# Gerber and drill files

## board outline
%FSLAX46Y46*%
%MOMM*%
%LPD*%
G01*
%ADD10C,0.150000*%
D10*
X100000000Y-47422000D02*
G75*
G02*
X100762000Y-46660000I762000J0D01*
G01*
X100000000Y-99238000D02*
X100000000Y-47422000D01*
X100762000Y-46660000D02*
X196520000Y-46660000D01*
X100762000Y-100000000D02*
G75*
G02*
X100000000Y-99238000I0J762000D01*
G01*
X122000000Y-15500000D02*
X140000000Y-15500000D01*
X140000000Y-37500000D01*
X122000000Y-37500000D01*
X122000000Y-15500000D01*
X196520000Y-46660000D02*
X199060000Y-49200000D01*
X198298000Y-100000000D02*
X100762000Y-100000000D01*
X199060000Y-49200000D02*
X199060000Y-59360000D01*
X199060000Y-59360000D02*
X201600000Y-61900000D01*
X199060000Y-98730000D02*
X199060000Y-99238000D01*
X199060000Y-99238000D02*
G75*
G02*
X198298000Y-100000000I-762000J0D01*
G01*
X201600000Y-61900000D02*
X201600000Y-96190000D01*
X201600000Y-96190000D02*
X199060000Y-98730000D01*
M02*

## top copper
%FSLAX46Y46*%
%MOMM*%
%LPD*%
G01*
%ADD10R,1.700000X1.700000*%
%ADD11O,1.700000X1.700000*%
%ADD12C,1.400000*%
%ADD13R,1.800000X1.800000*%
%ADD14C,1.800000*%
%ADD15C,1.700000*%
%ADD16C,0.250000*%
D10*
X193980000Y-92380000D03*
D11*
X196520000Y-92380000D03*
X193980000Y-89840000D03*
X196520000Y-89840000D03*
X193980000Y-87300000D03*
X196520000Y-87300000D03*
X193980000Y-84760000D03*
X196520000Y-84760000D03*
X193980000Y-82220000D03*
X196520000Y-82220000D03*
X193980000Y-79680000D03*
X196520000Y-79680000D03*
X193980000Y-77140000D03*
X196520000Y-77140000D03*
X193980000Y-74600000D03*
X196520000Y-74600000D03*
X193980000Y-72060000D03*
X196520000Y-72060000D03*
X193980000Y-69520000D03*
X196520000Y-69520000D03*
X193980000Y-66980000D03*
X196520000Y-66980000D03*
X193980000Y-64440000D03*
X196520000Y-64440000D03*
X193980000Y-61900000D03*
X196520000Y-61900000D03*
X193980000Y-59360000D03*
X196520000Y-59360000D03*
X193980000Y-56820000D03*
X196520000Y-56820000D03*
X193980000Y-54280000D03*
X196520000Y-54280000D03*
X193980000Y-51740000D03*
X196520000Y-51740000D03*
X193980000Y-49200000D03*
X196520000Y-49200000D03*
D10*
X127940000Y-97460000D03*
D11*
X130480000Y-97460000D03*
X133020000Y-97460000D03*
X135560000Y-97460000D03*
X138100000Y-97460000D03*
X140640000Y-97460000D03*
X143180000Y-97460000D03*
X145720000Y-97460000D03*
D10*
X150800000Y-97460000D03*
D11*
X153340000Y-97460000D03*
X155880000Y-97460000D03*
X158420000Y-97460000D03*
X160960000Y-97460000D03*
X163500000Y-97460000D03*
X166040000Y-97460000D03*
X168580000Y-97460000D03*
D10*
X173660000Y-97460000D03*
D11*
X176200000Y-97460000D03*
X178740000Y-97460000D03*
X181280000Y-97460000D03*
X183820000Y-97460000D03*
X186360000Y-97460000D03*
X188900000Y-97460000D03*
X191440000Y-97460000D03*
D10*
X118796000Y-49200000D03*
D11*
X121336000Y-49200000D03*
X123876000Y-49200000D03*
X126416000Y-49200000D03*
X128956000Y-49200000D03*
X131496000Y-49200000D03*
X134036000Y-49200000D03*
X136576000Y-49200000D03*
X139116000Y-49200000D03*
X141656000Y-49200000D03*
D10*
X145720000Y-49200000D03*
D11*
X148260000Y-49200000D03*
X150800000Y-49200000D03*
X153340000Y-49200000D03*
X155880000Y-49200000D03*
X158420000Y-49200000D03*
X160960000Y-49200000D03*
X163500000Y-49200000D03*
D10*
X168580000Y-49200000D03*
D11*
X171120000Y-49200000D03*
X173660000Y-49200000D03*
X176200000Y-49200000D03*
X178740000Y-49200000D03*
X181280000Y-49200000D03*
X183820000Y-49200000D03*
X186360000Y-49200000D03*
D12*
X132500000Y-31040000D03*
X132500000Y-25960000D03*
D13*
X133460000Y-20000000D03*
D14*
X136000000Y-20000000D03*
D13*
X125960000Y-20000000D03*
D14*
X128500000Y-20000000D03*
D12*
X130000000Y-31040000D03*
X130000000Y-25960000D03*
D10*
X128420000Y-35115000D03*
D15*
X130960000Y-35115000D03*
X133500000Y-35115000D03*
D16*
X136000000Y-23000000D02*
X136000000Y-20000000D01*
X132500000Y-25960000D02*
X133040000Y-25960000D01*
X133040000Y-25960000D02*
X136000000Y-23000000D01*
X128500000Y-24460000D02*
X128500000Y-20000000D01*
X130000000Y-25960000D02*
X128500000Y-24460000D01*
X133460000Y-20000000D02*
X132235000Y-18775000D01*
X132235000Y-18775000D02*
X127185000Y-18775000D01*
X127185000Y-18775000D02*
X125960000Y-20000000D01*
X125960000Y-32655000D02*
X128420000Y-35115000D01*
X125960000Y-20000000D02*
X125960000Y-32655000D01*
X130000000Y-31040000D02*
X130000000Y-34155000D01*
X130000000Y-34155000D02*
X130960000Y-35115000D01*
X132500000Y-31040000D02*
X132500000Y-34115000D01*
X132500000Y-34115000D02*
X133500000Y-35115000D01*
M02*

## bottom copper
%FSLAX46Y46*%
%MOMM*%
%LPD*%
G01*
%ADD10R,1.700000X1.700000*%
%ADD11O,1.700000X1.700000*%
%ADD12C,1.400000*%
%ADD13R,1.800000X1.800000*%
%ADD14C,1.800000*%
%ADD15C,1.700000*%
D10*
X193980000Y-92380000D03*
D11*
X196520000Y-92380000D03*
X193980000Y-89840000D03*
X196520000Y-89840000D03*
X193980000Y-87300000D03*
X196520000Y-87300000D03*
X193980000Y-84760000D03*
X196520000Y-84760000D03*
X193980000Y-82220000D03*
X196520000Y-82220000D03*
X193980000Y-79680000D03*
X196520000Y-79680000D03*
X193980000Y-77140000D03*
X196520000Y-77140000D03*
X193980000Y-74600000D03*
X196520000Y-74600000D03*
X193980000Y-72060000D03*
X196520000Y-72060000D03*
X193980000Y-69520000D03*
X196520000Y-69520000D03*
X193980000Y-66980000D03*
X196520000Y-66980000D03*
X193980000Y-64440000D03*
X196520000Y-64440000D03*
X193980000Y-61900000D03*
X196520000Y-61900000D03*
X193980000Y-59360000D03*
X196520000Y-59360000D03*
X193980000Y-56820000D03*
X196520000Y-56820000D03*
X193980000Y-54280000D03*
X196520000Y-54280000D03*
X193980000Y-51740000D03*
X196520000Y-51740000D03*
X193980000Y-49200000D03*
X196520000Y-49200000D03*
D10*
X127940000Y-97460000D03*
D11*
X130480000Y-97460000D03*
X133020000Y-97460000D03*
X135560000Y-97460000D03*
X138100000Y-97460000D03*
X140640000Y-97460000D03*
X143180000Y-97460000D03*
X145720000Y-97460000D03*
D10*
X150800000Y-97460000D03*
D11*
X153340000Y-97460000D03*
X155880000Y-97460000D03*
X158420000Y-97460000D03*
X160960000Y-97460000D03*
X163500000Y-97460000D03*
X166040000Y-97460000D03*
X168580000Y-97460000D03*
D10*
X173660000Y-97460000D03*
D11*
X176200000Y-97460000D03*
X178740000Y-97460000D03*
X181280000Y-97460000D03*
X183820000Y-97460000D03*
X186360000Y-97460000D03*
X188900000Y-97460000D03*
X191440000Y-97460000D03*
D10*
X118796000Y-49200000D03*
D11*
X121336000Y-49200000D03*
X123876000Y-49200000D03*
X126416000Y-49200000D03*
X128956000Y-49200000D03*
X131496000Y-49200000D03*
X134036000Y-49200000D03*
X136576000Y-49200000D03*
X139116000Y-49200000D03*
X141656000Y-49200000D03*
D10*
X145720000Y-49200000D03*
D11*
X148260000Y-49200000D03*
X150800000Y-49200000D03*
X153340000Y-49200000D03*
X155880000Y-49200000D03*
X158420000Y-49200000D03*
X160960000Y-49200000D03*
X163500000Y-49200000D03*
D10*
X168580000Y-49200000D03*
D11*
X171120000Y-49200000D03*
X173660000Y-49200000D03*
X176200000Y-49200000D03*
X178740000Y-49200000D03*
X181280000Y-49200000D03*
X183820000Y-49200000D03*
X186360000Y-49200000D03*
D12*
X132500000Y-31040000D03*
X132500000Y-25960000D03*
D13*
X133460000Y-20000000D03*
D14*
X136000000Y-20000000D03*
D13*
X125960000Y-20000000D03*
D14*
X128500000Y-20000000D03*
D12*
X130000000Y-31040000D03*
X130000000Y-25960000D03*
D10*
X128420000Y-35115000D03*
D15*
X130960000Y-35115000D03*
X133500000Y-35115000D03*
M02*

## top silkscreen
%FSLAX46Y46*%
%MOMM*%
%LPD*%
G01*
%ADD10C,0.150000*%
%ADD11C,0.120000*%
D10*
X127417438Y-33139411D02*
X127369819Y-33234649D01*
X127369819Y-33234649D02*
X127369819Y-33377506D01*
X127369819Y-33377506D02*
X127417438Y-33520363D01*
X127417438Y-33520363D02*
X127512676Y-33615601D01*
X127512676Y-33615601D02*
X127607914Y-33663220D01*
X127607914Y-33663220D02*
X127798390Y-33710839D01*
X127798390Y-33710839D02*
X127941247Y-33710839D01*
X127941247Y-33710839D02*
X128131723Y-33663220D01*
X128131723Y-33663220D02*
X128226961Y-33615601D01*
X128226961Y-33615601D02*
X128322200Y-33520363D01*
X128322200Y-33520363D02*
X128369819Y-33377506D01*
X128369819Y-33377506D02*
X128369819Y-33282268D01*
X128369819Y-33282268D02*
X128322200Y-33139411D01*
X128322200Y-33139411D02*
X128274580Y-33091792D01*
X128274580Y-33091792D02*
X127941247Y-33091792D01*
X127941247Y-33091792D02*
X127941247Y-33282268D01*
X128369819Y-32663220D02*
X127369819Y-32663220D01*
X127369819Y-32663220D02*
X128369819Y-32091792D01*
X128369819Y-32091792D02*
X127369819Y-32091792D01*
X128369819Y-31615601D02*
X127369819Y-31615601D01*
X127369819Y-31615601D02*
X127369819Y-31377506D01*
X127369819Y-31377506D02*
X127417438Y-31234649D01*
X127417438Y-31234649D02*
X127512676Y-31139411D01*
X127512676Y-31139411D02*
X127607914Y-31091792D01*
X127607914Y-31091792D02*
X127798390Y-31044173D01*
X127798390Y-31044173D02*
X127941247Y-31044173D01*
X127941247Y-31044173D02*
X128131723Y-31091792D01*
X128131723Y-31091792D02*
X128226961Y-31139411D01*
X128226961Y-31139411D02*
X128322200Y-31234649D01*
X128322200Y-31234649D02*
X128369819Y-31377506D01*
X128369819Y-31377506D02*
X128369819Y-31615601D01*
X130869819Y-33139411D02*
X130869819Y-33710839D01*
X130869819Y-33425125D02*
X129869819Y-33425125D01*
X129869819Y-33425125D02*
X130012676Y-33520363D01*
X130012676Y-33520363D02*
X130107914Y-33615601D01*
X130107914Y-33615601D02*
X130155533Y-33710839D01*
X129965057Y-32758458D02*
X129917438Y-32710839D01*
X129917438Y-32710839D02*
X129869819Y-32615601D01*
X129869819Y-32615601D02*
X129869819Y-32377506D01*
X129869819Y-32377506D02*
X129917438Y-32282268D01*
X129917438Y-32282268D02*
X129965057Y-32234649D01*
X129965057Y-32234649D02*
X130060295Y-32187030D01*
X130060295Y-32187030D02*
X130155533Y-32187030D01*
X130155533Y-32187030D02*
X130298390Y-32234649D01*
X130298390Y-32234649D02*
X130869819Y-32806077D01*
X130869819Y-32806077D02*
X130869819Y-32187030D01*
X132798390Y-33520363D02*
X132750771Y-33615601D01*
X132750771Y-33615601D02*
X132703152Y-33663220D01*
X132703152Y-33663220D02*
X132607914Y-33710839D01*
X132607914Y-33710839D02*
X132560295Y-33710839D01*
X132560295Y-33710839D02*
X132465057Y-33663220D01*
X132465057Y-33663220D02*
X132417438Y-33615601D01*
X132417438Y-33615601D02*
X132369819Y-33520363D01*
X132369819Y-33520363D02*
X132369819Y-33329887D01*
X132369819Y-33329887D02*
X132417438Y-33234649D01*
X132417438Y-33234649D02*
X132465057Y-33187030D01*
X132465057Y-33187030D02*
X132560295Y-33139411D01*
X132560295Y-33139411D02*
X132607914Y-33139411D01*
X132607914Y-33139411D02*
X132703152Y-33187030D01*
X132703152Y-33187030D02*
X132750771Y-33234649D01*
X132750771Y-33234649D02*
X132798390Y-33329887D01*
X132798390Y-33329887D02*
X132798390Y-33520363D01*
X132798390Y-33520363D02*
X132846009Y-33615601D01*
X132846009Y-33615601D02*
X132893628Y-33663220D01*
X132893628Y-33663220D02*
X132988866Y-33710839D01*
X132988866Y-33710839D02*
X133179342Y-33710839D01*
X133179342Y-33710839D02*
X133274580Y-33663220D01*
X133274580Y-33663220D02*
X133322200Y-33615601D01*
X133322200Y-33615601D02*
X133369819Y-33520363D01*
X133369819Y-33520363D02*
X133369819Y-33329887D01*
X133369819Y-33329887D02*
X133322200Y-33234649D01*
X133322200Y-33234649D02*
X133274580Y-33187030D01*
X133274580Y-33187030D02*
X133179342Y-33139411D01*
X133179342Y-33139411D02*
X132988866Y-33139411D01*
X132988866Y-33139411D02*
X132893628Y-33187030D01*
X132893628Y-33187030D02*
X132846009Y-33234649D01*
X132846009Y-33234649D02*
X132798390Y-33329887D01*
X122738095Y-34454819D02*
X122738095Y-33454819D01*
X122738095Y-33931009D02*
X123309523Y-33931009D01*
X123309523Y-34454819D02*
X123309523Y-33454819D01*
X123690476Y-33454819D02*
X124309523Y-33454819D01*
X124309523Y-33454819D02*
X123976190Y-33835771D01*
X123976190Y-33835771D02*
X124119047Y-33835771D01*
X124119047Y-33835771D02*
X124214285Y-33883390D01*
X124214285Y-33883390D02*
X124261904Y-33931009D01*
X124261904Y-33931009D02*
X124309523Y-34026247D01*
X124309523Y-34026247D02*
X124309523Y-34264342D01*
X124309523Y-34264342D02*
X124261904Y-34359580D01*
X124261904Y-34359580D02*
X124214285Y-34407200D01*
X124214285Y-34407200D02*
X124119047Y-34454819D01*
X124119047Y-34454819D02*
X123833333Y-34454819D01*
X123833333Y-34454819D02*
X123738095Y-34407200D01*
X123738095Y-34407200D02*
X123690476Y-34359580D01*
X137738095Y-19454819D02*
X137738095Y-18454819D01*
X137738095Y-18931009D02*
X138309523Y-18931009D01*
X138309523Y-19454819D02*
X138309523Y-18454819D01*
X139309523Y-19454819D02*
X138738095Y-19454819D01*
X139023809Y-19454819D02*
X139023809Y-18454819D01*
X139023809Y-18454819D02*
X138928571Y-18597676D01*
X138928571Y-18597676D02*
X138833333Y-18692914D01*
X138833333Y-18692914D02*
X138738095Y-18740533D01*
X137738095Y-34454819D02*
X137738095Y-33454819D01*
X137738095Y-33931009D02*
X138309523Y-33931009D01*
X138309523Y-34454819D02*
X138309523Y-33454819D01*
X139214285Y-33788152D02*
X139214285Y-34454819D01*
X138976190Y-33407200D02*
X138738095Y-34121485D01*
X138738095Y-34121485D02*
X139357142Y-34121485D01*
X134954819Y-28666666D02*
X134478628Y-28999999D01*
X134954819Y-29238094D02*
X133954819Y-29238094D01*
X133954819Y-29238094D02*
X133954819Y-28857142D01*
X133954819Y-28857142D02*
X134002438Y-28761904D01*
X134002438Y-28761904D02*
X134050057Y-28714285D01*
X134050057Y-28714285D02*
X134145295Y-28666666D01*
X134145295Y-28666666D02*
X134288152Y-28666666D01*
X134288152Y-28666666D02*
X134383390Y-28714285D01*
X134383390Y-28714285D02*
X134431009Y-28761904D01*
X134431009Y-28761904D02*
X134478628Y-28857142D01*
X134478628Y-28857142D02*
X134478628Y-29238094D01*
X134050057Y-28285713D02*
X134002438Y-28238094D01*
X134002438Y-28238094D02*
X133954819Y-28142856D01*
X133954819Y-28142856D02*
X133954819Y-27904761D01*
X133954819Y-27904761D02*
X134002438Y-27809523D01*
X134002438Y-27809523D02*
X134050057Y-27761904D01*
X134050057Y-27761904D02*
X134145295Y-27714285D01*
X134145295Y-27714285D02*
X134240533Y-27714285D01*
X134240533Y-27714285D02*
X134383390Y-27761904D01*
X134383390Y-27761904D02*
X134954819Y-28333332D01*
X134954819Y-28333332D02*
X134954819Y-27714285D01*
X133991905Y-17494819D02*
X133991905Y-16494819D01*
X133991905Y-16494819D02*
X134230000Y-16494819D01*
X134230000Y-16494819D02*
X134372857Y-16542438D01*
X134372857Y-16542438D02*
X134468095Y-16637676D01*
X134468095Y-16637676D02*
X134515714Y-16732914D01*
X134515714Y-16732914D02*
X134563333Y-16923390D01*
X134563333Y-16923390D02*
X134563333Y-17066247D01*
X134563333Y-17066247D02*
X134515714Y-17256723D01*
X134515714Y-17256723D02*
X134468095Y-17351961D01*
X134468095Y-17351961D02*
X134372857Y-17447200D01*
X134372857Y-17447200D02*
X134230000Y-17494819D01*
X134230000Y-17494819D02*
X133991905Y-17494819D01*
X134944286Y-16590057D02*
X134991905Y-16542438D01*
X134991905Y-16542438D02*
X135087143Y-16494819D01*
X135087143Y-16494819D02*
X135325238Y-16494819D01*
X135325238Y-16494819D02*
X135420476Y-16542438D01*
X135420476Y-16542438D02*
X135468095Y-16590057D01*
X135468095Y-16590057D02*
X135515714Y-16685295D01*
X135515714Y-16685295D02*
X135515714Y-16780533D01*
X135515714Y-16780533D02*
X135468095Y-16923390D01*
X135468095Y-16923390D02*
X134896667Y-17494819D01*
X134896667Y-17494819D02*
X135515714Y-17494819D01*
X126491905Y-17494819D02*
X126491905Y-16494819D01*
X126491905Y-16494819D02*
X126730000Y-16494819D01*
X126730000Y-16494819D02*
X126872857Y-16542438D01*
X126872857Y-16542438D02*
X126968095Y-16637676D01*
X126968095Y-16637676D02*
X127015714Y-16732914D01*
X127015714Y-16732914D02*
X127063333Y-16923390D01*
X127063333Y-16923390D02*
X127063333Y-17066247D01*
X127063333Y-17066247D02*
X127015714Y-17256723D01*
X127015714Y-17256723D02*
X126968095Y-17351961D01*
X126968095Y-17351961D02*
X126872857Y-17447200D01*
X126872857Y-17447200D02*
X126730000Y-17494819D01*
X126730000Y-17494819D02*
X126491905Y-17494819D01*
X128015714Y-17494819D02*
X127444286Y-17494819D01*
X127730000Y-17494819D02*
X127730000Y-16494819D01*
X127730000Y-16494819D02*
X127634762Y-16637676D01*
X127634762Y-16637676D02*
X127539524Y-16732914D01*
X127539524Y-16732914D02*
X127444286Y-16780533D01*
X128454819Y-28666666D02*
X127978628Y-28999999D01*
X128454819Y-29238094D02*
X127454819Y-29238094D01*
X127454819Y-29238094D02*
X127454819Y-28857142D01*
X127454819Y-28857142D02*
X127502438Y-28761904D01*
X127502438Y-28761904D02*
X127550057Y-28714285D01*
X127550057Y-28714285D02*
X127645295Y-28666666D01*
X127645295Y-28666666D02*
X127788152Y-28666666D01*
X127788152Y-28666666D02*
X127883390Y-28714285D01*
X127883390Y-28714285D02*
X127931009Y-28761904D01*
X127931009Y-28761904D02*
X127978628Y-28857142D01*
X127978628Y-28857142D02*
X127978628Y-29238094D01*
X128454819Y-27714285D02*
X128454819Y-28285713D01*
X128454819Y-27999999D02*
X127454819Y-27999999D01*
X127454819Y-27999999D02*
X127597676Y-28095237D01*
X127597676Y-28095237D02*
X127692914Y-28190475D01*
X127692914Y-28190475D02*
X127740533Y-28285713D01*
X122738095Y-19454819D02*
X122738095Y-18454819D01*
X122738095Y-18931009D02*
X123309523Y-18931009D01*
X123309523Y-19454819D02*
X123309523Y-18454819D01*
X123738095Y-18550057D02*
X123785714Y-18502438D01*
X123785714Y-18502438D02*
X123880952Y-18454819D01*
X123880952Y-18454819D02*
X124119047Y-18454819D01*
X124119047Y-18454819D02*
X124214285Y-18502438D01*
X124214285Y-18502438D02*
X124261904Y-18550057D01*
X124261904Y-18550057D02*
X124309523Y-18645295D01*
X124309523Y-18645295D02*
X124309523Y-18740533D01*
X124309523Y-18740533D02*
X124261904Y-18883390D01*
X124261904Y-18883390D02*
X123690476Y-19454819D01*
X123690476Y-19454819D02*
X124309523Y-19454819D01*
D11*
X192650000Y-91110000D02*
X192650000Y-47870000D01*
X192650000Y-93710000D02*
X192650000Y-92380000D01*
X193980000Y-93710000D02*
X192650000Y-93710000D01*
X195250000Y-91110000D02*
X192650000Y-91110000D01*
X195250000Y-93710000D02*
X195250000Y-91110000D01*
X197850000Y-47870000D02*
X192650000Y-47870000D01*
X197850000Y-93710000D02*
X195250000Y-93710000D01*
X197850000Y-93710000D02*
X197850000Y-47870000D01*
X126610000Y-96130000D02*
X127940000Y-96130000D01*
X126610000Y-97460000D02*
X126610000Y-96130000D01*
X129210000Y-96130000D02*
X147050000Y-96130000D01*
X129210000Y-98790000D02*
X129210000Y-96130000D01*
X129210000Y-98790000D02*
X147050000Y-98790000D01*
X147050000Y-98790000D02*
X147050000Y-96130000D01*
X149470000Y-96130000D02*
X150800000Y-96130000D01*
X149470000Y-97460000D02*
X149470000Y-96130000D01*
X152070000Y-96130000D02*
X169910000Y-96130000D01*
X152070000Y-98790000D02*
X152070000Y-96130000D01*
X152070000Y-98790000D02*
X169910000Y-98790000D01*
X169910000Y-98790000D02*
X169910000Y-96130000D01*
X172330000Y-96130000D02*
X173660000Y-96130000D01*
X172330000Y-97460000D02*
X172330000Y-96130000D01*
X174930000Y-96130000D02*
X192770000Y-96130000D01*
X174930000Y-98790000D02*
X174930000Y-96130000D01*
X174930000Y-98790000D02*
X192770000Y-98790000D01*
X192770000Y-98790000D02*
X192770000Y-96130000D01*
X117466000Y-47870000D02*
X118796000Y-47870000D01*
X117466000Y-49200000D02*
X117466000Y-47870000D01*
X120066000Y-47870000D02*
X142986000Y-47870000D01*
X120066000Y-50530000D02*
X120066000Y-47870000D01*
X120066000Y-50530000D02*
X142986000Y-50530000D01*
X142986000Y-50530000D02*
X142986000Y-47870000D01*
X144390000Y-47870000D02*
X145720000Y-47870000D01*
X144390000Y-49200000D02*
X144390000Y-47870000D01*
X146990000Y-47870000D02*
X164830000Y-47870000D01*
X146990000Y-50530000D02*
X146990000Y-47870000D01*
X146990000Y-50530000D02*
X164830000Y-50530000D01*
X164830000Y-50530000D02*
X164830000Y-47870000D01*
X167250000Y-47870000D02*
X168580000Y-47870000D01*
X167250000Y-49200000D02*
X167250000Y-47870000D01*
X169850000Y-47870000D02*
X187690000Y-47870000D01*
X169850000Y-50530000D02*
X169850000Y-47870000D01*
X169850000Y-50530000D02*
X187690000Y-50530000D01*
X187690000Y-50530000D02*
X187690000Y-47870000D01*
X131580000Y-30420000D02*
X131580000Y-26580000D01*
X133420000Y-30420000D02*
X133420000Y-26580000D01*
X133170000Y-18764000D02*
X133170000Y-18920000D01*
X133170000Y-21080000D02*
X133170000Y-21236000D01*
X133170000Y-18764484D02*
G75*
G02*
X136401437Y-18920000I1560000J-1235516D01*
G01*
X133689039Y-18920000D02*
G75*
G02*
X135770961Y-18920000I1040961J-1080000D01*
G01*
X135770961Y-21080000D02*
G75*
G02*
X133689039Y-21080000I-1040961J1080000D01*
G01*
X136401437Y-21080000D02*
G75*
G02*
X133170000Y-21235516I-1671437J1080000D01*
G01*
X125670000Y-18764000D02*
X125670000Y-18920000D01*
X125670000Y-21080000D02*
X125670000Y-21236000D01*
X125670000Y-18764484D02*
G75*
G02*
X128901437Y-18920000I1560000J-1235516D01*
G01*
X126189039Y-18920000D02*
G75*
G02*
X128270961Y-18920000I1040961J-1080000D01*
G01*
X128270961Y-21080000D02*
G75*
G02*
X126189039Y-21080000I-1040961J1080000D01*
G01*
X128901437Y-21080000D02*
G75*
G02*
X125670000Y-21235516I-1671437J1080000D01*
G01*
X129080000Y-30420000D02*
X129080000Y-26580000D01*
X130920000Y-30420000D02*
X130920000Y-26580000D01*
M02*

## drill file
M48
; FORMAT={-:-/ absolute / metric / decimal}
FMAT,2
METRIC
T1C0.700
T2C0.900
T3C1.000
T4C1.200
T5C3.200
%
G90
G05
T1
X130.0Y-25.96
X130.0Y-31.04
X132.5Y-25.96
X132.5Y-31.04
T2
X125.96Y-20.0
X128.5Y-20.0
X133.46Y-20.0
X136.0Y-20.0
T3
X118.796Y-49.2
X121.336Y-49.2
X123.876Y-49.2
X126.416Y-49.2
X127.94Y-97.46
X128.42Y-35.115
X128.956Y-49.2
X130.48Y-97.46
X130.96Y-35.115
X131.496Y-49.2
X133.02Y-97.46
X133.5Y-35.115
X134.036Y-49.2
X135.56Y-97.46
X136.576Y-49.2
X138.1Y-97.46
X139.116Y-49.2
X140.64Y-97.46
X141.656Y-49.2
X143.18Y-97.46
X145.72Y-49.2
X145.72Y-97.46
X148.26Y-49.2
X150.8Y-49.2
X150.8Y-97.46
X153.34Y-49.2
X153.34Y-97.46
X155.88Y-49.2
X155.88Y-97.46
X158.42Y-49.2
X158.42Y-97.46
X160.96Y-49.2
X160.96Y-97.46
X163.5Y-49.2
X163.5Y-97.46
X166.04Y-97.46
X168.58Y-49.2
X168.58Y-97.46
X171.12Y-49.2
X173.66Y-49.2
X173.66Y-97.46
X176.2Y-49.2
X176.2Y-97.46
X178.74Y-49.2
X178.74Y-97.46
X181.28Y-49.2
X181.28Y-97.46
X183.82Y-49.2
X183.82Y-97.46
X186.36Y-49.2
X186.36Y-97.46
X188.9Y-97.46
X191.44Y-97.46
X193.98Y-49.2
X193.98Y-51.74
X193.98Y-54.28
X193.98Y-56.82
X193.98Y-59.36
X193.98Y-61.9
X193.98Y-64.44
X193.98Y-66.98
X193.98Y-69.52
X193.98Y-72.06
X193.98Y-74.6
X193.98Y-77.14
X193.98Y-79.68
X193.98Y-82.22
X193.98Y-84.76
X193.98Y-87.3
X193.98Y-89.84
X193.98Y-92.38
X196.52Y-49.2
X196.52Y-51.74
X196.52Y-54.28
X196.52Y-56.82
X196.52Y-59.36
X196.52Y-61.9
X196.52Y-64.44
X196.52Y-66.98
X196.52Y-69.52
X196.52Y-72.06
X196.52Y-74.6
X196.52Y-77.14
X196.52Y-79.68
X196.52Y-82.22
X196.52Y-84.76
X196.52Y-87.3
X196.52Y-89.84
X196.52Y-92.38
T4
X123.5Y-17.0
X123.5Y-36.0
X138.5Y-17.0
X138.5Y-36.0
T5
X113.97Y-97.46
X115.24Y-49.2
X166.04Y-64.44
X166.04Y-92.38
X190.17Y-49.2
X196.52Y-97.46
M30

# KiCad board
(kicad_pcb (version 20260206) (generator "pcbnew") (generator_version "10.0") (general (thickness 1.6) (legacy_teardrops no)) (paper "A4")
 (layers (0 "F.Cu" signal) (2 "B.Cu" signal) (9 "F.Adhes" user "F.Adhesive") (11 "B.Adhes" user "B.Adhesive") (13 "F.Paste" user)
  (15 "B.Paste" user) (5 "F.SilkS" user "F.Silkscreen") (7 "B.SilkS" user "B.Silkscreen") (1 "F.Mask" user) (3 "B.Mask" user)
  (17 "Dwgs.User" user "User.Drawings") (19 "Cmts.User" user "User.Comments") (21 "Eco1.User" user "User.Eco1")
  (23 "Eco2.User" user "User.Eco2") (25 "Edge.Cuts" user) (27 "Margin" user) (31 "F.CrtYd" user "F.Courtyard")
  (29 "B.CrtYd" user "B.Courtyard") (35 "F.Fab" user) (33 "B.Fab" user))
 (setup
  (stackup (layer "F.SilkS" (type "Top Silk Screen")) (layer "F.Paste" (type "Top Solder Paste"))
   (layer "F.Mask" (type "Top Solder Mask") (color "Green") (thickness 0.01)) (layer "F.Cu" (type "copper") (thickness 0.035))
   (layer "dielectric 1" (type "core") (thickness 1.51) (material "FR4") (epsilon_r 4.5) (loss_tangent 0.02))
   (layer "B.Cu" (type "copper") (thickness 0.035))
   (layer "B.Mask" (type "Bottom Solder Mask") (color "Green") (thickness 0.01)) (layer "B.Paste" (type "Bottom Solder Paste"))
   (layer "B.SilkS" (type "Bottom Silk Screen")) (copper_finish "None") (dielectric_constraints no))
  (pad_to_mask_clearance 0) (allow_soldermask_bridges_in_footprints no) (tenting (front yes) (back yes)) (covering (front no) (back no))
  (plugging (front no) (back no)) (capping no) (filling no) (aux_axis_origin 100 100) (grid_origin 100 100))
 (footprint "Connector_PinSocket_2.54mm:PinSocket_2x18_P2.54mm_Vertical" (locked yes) (layer "F.Cu") (at 193.98 92.38 180)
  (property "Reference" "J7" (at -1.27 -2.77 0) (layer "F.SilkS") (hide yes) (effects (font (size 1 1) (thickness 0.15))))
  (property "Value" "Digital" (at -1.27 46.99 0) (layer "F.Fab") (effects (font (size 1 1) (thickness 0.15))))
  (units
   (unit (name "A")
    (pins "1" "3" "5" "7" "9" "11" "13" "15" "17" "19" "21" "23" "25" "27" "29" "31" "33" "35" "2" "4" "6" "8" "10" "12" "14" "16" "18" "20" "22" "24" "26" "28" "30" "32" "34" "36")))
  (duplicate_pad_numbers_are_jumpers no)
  (fp_line (start 1.33 1.27) (end 1.33 44.51) (stroke (width 0.12) (type solid)) (layer "F.SilkS"))
  (fp_line (start 1.33 -1.33) (end 1.33 0) (stroke (width 0.12) (type solid)) (layer "F.SilkS"))
  (fp_line (start 0 -1.33) (end 1.33 -1.33) (stroke (width 0.12) (type solid)) (layer "F.SilkS"))
  (fp_line (start -1.27 1.27) (end 1.33 1.27) (stroke (width 0.12) (type solid)) (layer "F.SilkS"))
  (fp_line (start -1.27 -1.33) (end -1.27 1.27) (stroke (width 0.12) (type solid)) (layer "F.SilkS"))
  (fp_line (start -3.87 44.51) (end 1.33 44.51) (stroke (width 0.12) (type solid)) (layer "F.SilkS"))
  (fp_line (start -3.87 -1.33) (end -1.27 -1.33) (stroke (width 0.12) (type solid)) (layer "F.SilkS"))
  (fp_line (start -3.87 -1.33) (end -3.87 44.51) (stroke (width 0.12) (type solid)) (layer "F.SilkS"))
  (pad "1" thru_hole rect (at 0 0 180) (size 1.7 1.7) (drill 1) (layers "*.Cu" "*.Mask") (remove_unused_layers no) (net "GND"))
  (pad "2" thru_hole oval (at -2.54 0 180) (size 1.7 1.7) (drill 1) (layers "*.Cu" "*.Mask") (remove_unused_layers no) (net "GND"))
  (pad "3" thru_hole oval (at 0 2.54 180) (size 1.7 1.7) (drill 1) (layers "*.Cu" "*.Mask") (remove_unused_layers no) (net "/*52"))
  (pad "4" thru_hole oval (at -2.54 2.54 180) (size 1.7 1.7) (drill 1) (layers "*.Cu" "*.Mask") (remove_unused_layers no) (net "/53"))
  (pad "5" thru_hole oval (at 0 5.08 180) (size 1.7 1.7) (drill 1) (layers "*.Cu" "*.Mask") (remove_unused_layers no) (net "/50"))
  (pad "6" thru_hole oval (at -2.54 5.08 180) (size 1.7 1.7) (drill 1) (layers "*.Cu" "*.Mask") (remove_unused_layers no) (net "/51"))
  (pad "7" thru_hole oval (at 0 7.62 180) (size 1.7 1.7) (drill 1) (layers "*.Cu" "*.Mask") (remove_unused_layers no) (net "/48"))
  (pad "8" thru_hole oval (at -2.54 7.62 180) (size 1.7 1.7) (drill 1) (layers "*.Cu" "*.Mask") (remove_unused_layers no) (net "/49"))
  (pad "9" thru_hole oval (at 0 10.16 180) (size 1.7 1.7) (drill 1) (layers "*.Cu" "*.Mask") (remove_unused_layers no) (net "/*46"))
  (pad "10" thru_hole oval (at -2.54 10.16 180) (size 1.7 1.7) (drill 1) (layers "*.Cu" "*.Mask") (remove_unused_layers no) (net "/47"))
  (pad "11" thru_hole oval (at 0 12.7 180) (size 1.7 1.7) (drill 1) (layers "*.Cu" "*.Mask") (remove_unused_layers no) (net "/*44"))
  (pad "12" thru_hole oval (at -2.54 12.7 180) (size 1.7 1.7) (drill 1) (layers "*.Cu" "*.Mask") (remove_unused_layers no) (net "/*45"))
  (pad "13" thru_hole oval (at 0 15.24 180) (size 1.7 1.7) (drill 1) (layers "*.Cu" "*.Mask") (remove_unused_layers no) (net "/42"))
  (pad "14" thru_hole oval (at -2.54 15.24 180) (size 1.7 1.7) (drill 1) (layers "*.Cu" "*.Mask") (remove_unused_layers no) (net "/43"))
  (pad "15" thru_hole oval (at 0 17.78 180) (size 1.7 1.7) (drill 1) (layers "*.Cu" "*.Mask") (remove_unused_layers no) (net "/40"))
  (pad "16" thru_hole oval (at -2.54 17.78 180) (size 1.7 1.7) (drill 1) (layers "*.Cu" "*.Mask") (remove_unused_layers no) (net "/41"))
  (pad "17" thru_hole oval (at 0 20.32 180) (size 1.7 1.7) (drill 1) (layers "*.Cu" "*.Mask") (remove_unused_layers no) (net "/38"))
  (pad "18" thru_hole oval (at -2.54 20.32 180) (size 1.7 1.7) (drill 1) (layers "*.Cu" "*.Mask") (remove_unused_layers no) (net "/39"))
  (pad "19" thru_hole oval (at 0 22.86 180) (size 1.7 1.7) (drill 1) (layers "*.Cu" "*.Mask") (remove_unused_layers no) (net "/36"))
  (pad "20" thru_hole oval (at -2.54 22.86 180) (size 1.7 1.7) (drill 1) (layers "*.Cu" "*.Mask") (remove_unused_layers no) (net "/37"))
  (pad "21" thru_hole oval (at 0 25.4 180) (size 1.7 1.7) (drill 1) (layers "*.Cu" "*.Mask") (remove_unused_layers no) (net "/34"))
  (pad "22" thru_hole oval (at -2.54 25.4 180) (size 1.7 1.7) (drill 1) (layers "*.Cu" "*.Mask") (remove_unused_layers no) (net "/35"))
  (pad "23" thru_hole oval (at 0 27.94 180) (size 1.7 1.7) (drill 1) (layers "*.Cu" "*.Mask") (remove_unused_layers no) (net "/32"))
  (pad "24" thru_hole oval (at -2.54 27.94 180) (size 1.7 1.7) (drill 1) (layers "*.Cu" "*.Mask") (remove_unused_layers no) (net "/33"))
  (pad "25" thru_hole oval (at 0 30.48 180) (size 1.7 1.7) (drill 1) (layers "*.Cu" "*.Mask") (remove_unused_layers no) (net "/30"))
  (pad "26" thru_hole oval (at -2.54 30.48 180) (size 1.7 1.7) (drill 1) (layers "*.Cu" "*.Mask") (remove_unused_layers no) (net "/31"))
  (pad "27" thru_hole oval (at 0 33.02 180) (size 1.7 1.7) (drill 1) (layers "*.Cu" "*.Mask") (remove_unused_layers no) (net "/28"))
  (pad "28" thru_hole oval (at -2.54 33.02 180) (size 1.7 1.7) (drill 1) (layers "*.Cu" "*.Mask") (remove_unused_layers no) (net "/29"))
  (pad "29" thru_hole oval (at 0 35.56 180) (size 1.7 1.7) (drill 1) (layers "*.Cu" "*.Mask") (remove_unused_layers no) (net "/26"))
  (pad "30" thru_hole oval (at -2.54 35.56 180) (size 1.7 1.7) (drill 1) (layers "*.Cu" "*.Mask") (remove_unused_layers no) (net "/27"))
  (pad "31" thru_hole oval (at 0 38.1 180) (size 1.7 1.7) (drill 1) (layers "*.Cu" "*.Mask") (remove_unused_layers no) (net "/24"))
  (pad "32" thru_hole oval (at -2.54 38.1 180) (size 1.7 1.7) (drill 1) (layers "*.Cu" "*.Mask") (remove_unused_layers no) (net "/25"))
  (pad "33" thru_hole oval (at 0 40.64 180) (size 1.7 1.7) (drill 1) (layers "*.Cu" "*.Mask") (remove_unused_layers no) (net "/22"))
  (pad "34" thru_hole oval (at -2.54 40.64 180) (size 1.7 1.7) (drill 1) (layers "*.Cu" "*.Mask") (remove_unused_layers no) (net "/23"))
  (pad "35" thru_hole oval (at 0 43.18 180) (size 1.7 1.7) (drill 1) (layers "*.Cu" "*.Mask") (remove_unused_layers no) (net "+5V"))
  (pad "36" thru_hole oval (at -2.54 43.18 180) (size 1.7 1.7) (drill 1) (layers "*.Cu" "*.Mask") (remove_unused_layers no) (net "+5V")))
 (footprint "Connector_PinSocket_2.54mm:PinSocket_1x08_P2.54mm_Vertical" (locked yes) (layer "F.Cu") (at 127.94 97.46 90)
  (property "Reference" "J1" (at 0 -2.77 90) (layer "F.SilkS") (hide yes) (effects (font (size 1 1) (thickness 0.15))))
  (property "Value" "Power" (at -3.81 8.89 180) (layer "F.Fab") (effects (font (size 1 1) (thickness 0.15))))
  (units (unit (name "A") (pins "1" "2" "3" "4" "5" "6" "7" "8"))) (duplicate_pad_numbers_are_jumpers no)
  (fp_line (start 1.33 -1.33) (end 1.33 0) (stroke (width 0.12) (type solid)) (layer "F.SilkS"))
  (fp_line (start 0 -1.33) (end 1.33 -1.33) (stroke (width 0.12) (type solid)) (layer "F.SilkS"))
  (fp_line (start 1.33 1.27) (end 1.33 19.11) (stroke (width 0.12) (type solid)) (layer "F.SilkS"))
  (fp_line (start -1.33 1.27) (end 1.33 1.27) (stroke (width 0.12) (type solid)) (layer "F.SilkS"))
  (fp_line (start -1.33 1.27) (end -1.33 19.11) (stroke (width 0.12) (type solid)) (layer "F.SilkS"))
  (fp_line (start -1.33 19.11) (end 1.33 19.11) (stroke (width 0.12) (type solid)) (layer "F.SilkS"))
  (pad "1" thru_hole rect (at 0 0 90) (size 1.7 1.7) (drill 1) (layers "*.Cu" "*.Mask") (remove_unused_layers no)
   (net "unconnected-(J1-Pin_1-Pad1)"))
  (pad "2" thru_hole oval (at 0 2.54 90) (size 1.7 1.7) (drill 1) (layers "*.Cu" "*.Mask") (remove_unused_layers no) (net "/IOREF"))
  (pad "3" thru_hole oval (at 0 5.08 90) (size 1.7 1.7) (drill 1) (layers "*.Cu" "*.Mask") (remove_unused_layers no) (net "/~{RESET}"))
  (pad "4" thru_hole oval (at 0 7.62 90) (size 1.7 1.7) (drill 1) (layers "*.Cu" "*.Mask") (remove_unused_layers no) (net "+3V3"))
  (pad "5" thru_hole oval (at 0 10.16 90) (size 1.7 1.7) (drill 1) (layers "*.Cu" "*.Mask") (remove_unused_layers no) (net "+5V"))
  (pad "6" thru_hole oval (at 0 12.7 90) (size 1.7 1.7) (drill 1) (layers "*.Cu" "*.Mask") (remove_unused_layers no) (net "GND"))
  (pad "7" thru_hole oval (at 0 15.24 90) (size 1.7 1.7) (drill 1) (layers "*.Cu" "*.Mask") (remove_unused_layers no) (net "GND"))
  (pad "8" thru_hole oval (at 0 17.78 90) (size 1.7 1.7) (drill 1) (layers "*.Cu" "*.Mask") (remove_unused_layers no) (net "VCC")))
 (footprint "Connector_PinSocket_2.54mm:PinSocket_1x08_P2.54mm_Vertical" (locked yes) (layer "F.Cu") (at 150.8 97.46 90)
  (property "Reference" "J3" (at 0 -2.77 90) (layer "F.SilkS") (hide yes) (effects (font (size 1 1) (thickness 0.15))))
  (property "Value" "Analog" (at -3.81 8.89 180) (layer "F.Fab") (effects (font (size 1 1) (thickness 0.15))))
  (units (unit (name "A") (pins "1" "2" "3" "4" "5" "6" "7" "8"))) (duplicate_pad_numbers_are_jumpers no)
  (fp_line (start 1.33 -1.33) (end 1.33 0) (stroke (width 0.12) (type solid)) (layer "F.SilkS"))
  (fp_line (start 0 -1.33) (end 1.33 -1.33) (stroke (width 0.12) (type solid)) (layer "F.SilkS"))
  (fp_line (start 1.33 1.27) (end 1.33 19.11) (stroke (width 0.12) (type solid)) (layer "F.SilkS"))
  (fp_line (start -1.33 1.27) (end 1.33 1.27) (stroke (width 0.12) (type solid)) (layer "F.SilkS"))
  (fp_line (start -1.33 1.27) (end -1.33 19.11) (stroke (width 0.12) (type solid)) (layer "F.SilkS"))
  (fp_line (start -1.33 19.11) (end 1.33 19.11) (stroke (width 0.12) (type solid)) (layer "F.SilkS"))
  (pad "1" thru_hole rect (at 0 0 90) (size 1.7 1.7) (drill 1) (layers "*.Cu" "*.Mask") (remove_unused_layers no) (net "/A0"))
  (pad "2" thru_hole oval (at 0 2.54 90) (size 1.7 1.7) (drill 1) (layers "*.Cu" "*.Mask") (remove_unused_layers no) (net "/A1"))
  (pad "3" thru_hole oval (at 0 5.08 90) (size 1.7 1.7) (drill 1) (layers "*.Cu" "*.Mask") (remove_unused_layers no) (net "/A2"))
  (pad "4" thru_hole oval (at 0 7.62 90) (size 1.7 1.7) (drill 1) (layers "*.Cu" "*.Mask") (remove_unused_layers no) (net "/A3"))
  (pad "5" thru_hole oval (at 0 10.16 90) (size 1.7 1.7) (drill 1) (layers "*.Cu" "*.Mask") (remove_unused_layers no) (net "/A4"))
  (pad "6" thru_hole oval (at 0 12.7 90) (size 1.7 1.7) (drill 1) (layers "*.Cu" "*.Mask") (remove_unused_layers no) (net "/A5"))
  (pad "7" thru_hole oval (at 0 15.24 90) (size 1.7 1.7) (drill 1) (layers "*.Cu" "*.Mask") (remove_unused_layers no) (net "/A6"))
  (pad "8" thru_hole oval (at 0 17.78 90) (size 1.7 1.7) (drill 1) (layers "*.Cu" "*.Mask") (remove_unused_layers no) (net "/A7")))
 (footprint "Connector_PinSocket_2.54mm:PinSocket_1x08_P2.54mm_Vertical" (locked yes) (layer "F.Cu") (at 173.66 97.46 90)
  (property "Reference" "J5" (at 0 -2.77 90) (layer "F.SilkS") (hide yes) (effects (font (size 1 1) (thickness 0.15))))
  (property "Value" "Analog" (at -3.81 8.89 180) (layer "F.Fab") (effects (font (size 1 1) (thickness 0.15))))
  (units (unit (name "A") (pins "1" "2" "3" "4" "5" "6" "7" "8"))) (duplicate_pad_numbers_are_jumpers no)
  (fp_line (start 1.33 -1.33) (end 1.33 0) (stroke (width 0.12) (type solid)) (layer "F.SilkS"))
  (fp_line (start 0 -1.33) (end 1.33 -1.33) (stroke (width 0.12) (type solid)) (layer "F.SilkS"))
  (fp_line (start 1.33 1.27) (end 1.33 19.11) (stroke (width 0.12) (type solid)) (layer "F.SilkS"))
  (fp_line (start -1.33 1.27) (end 1.33 1.27) (stroke (width 0.12) (type solid)) (layer "F.SilkS"))
  (fp_line (start -1.33 1.27) (end -1.33 19.11) (stroke (width 0.12) (type solid)) (layer "F.SilkS"))
  (fp_line (start -1.33 19.11) (end 1.33 19.11) (stroke (width 0.12) (type solid)) (layer "F.SilkS"))
  (pad "1" thru_hole rect (at 0 0 90) (size 1.7 1.7) (drill 1) (layers "*.Cu" "*.Mask") (remove_unused_layers no) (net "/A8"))
  (pad "2" thru_hole oval (at 0 2.54 90) (size 1.7 1.7) (drill 1) (layers "*.Cu" "*.Mask") (remove_unused_layers no) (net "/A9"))
  (pad "3" thru_hole oval (at 0 5.08 90) (size 1.7 1.7) (drill 1) (layers "*.Cu" "*.Mask") (remove_unused_layers no) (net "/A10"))
  (pad "4" thru_hole oval (at 0 7.62 90) (size 1.7 1.7) (drill 1) (layers "*.Cu" "*.Mask") (remove_unused_layers no) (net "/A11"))
  (pad "5" thru_hole oval (at 0 10.16 90) (size 1.7 1.7) (drill 1) (layers "*.Cu" "*.Mask") (remove_unused_layers no) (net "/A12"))
  (pad "6" thru_hole oval (at 0 12.7 90) (size 1.7 1.7) (drill 1) (layers "*.Cu" "*.Mask") (remove_unused_layers no) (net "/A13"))
  (pad "7" thru_hole oval (at 0 15.24 90) (size 1.7 1.7) (drill 1) (layers "*.Cu" "*.Mask") (remove_unused_layers no) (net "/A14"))
  (pad "8" thru_hole oval (at 0 17.78 90) (size 1.7 1.7) (drill 1) (layers "*.Cu" "*.Mask") (remove_unused_layers no) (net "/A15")))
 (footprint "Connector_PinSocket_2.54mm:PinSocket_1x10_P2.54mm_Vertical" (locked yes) (layer "F.Cu") (at 118.796 49.2 90)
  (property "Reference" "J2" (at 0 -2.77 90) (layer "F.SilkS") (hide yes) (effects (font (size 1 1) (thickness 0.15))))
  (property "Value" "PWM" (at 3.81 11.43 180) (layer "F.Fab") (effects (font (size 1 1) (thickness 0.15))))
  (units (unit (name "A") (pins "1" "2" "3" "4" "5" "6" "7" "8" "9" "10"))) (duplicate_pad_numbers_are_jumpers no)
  (fp_line (start 1.33 -1.33) (end 1.33 0) (stroke (width 0.12) (type solid)) (layer "F.SilkS"))
  (fp_line (start 0 -1.33) (end 1.33 -1.33) (stroke (width 0.12) (type solid)) (layer "F.SilkS"))
  (fp_line (start 1.33 1.27) (end 1.33 24.19) (stroke (width 0.12) (type solid)) (layer "F.SilkS"))
  (fp_line (start -1.33 1.27) (end 1.33 1.27) (stroke (width 0.12) (type solid)) (layer "F.SilkS"))
  (fp_line (start -1.33 1.27) (end -1.33 24.19) (stroke (width 0.12) (type solid)) (layer "F.SilkS"))
  (fp_line (start -1.33 24.19) (end 1.33 24.19) (stroke (width 0.12) (type solid)) (layer "F.SilkS"))
  (pad "1" thru_hole rect (at 0 0 90) (size 1.7 1.7) (drill 1) (layers "*.Cu" "*.Mask") (remove_unused_layers no) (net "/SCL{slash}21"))
  (pad "2" thru_hole oval (at 0 2.54 90) (size 1.7 1.7) (drill 1) (layers "*.Cu" "*.Mask") (remove_unused_layers no) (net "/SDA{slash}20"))
  (pad "3" thru_hole oval (at 0 5.08 90) (size 1.7 1.7) (drill 1) (layers "*.Cu" "*.Mask") (remove_unused_layers no) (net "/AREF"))
  (pad "4" thru_hole oval (at 0 7.62 90) (size 1.7 1.7) (drill 1) (layers "*.Cu" "*.Mask") (remove_unused_layers no) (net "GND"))
  (pad "5" thru_hole oval (at 0 10.16 90) (size 1.7 1.7) (drill 1) (layers "*.Cu" "*.Mask") (remove_unused_layers no) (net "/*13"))
  (pad "6" thru_hole oval (at 0 12.7 90) (size 1.7 1.7) (drill 1) (layers "*.Cu" "*.Mask") (remove_unused_layers no)
   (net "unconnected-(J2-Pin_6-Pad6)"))
  (pad "7" thru_hole oval (at 0 15.24 90) (size 1.7 1.7) (drill 1) (layers "*.Cu" "*.Mask") (remove_unused_layers no) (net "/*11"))
  (pad "8" thru_hole oval (at 0 17.78 90) (size 1.7 1.7) (drill 1) (layers "*.Cu" "*.Mask") (remove_unused_layers no)
   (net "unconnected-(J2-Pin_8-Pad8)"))
  (pad "9" thru_hole oval (at 0 20.32 90) (size 1.7 1.7) (drill 1) (layers "*.Cu" "*.Mask") (remove_unused_layers no) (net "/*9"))
  (pad "10" thru_hole oval (at 0 22.86 90) (size 1.7 1.7) (drill 1) (layers "*.Cu" "*.Mask") (remove_unused_layers no)
   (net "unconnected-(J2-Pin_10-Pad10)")))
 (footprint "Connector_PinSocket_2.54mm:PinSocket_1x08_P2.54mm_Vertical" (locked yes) (layer "F.Cu") (at 145.72 49.2 90)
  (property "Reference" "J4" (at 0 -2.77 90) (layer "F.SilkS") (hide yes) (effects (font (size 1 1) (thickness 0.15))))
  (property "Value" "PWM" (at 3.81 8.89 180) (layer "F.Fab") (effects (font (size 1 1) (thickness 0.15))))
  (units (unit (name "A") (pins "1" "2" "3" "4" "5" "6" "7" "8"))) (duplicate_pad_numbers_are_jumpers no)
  (fp_line (start 1.33 -1.33) (end 1.33 0) (stroke (width 0.12) (type solid)) (layer "F.SilkS"))
  (fp_line (start 0 -1.33) (end 1.33 -1.33) (stroke (width 0.12) (type solid)) (layer "F.SilkS"))
  (fp_line (start 1.33 1.27) (end 1.33 19.11) (stroke (width 0.12) (type solid)) (layer "F.SilkS"))
  (fp_line (start -1.33 1.27) (end 1.33 1.27) (stroke (width 0.12) (type solid)) (layer "F.SilkS"))
  (fp_line (start -1.33 1.27) (end -1.33 19.11) (stroke (width 0.12) (type solid)) (layer "F.SilkS"))
  (fp_line (start -1.33 19.11) (end 1.33 19.11) (stroke (width 0.12) (type solid)) (layer "F.SilkS"))
  (pad "1" thru_hole rect (at 0 0 90) (size 1.7 1.7) (drill 1) (layers "*.Cu" "*.Mask") (remove_unused_layers no) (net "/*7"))
  (pad "2" thru_hole oval (at 0 2.54 90) (size 1.7 1.7) (drill 1) (layers "*.Cu" "*.Mask") (remove_unused_layers no) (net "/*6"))
  (pad "3" thru_hole oval (at 0 5.08 90) (size 1.7 1.7) (drill 1) (layers "*.Cu" "*.Mask") (remove_unused_layers no) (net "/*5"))
  (pad "4" thru_hole oval (at 0 7.62 90) (size 1.7 1.7) (drill 1) (layers "*.Cu" "*.Mask") (remove_unused_layers no) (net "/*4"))
  (pad "5" thru_hole oval (at 0 10.16 90) (size 1.7 1.7) (drill 1) (layers "*.Cu" "*.Mask") (remove_unused_layers no) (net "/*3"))
  (pad "6" thru_hole oval (at 0 12.7 90) (size 1.7 1.7) (drill 1) (layers "*.Cu" "*.Mask") (remove_unused_layers no) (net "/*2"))
  (pad "7" thru_hole oval (at 0 15.24 90) (size 1.7 1.7) (drill 1) (layers "*.Cu" "*.Mask") (remove_unused_layers no) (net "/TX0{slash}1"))
  (pad "8" thru_hole oval (at 0 17.78 90) (size 1.7 1.7) (drill 1) (layers "*.Cu" "*.Mask") (remove_unused_layers no) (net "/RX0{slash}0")))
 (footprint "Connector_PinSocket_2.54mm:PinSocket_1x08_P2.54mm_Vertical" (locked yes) (layer "F.Cu") (at 168.58 49.2 90)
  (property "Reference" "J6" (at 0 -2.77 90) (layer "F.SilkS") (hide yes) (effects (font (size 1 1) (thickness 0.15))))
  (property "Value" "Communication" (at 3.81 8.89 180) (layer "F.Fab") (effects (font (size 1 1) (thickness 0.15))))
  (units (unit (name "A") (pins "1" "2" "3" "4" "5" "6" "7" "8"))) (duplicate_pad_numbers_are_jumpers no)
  (fp_line (start 1.33 -1.33) (end 1.33 0) (stroke (width 0.12) (type solid)) (layer "F.SilkS"))
  (fp_line (start 0 -1.33) (end 1.33 -1.33) (stroke (width 0.12) (type solid)) (layer "F.SilkS"))
  (fp_line (start 1.33 1.27) (end 1.33 19.11) (stroke (width 0.12) (type solid)) (layer "F.SilkS"))
  (fp_line (start -1.33 1.27) (end 1.33 1.27) (stroke (width 0.12) (type solid)) (layer "F.SilkS"))
  (fp_line (start -1.33 1.27) (end -1.33 19.11) (stroke (width 0.12) (type solid)) (layer "F.SilkS"))
  (fp_line (start -1.33 19.11) (end 1.33 19.11) (stroke (width 0.12) (type solid)) (layer "F.SilkS"))
  (pad "1" thru_hole rect (at 0 0 90) (size 1.7 1.7) (drill 1) (layers "*.Cu" "*.Mask") (remove_unused_layers no) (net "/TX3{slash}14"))
  (pad "2" thru_hole oval (at 0 2.54 90) (size 1.7 1.7) (drill 1) (layers "*.Cu" "*.Mask") (remove_unused_layers no) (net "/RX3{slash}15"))
  (pad "3" thru_hole oval (at 0 5.08 90) (size 1.7 1.7) (drill 1) (layers "*.Cu" "*.Mask") (remove_unused_layers no) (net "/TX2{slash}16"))
  (pad "4" thru_hole oval (at 0 7.62 90) (size 1.7 1.7) (drill 1) (layers "*.Cu" "*.Mask") (remove_unused_layers no) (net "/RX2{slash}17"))
  (pad "5" thru_hole oval (at 0 10.16 90) (size 1.7 1.7) (drill 1) (layers "*.Cu" "*.Mask") (remove_unused_layers no) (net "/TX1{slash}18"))
  (pad "6" thru_hole oval (at 0 12.7 90) (size 1.7 1.7) (drill 1) (layers "*.Cu" "*.Mask") (remove_unused_layers no) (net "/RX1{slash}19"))
  (pad "7" thru_hole oval (at 0 15.24 90) (size 1.7 1.7) (drill 1) (layers "*.Cu" "*.Mask") (remove_unused_layers no) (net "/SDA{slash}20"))
  (pad "8" thru_hole oval (at 0 17.78 90) (size 1.7 1.7) (drill 1) (layers "*.Cu" "*.Mask") (remove_unused_layers no) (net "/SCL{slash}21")))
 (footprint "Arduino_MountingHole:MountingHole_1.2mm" (layer "F.Cu") (at 123.5 36)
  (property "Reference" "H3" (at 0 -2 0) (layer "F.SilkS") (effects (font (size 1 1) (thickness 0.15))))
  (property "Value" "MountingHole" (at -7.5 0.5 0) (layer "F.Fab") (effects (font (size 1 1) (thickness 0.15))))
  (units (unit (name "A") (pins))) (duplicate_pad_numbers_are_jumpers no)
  (pad "" np_thru_hole circle (at 0 0) (size 1.2 1.2) (drill 1.2) (layers "*.Cu" "*.Mask")))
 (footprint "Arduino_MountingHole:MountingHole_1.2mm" (layer "F.Cu") (at 138.5 17)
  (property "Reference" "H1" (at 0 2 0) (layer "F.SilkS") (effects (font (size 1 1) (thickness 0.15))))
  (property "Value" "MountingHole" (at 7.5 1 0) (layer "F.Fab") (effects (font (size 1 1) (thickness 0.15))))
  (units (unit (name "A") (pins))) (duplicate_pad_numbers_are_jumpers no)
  (pad "" np_thru_hole circle (at 0 0) (size 1.2 1.2) (drill 1.2) (layers "*.Cu" "*.Mask")))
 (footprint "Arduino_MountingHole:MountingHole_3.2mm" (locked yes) (layer "F.Cu") (at 196.52 97.46)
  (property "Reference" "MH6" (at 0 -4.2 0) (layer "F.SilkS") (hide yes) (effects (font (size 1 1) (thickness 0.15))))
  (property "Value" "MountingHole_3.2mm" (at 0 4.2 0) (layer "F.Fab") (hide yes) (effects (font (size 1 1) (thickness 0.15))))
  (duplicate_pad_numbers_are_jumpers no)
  (pad "" np_thru_hole circle (at 0 0) (size 3.2 3.2) (drill 3.2) (layers "*.Cu" "*.Mask")))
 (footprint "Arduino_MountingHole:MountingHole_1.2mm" (layer "F.Cu") (at 138.5 36)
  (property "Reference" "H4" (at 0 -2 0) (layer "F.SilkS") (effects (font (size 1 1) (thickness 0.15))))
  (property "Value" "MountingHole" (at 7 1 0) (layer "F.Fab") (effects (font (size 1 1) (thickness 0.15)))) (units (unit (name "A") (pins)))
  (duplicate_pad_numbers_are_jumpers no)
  (pad "" np_thru_hole circle (at 0 0) (size 1.2 1.2) (drill 1.2) (layers "*.Cu" "*.Mask")))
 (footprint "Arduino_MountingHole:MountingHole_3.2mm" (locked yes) (layer "F.Cu") (at 115.24 49.2)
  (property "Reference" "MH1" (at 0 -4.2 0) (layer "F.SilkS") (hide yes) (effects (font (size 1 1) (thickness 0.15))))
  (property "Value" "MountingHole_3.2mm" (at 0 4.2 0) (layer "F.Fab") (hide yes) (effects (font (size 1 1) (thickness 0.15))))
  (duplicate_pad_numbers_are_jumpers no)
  (pad "" np_thru_hole circle (at 0 0) (size 3.2 3.2) (drill 3.2) (layers "*.Cu" "*.Mask")))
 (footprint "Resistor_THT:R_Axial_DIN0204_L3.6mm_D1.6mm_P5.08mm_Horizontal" (layer "F.Cu") (at 132.5 31.04 90)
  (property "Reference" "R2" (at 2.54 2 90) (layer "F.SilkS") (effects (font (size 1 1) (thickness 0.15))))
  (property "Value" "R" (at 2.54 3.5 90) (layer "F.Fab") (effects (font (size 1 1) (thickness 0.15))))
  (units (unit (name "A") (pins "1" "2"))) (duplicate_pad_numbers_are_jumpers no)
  (fp_line (start 0.62 -0.92) (end 4.46 -0.92) (stroke (width 0.12) (type solid)) (layer "F.SilkS"))
  (fp_line (start 0.62 0.92) (end 4.46 0.92) (stroke (width 0.12) (type solid)) (layer "F.SilkS"))
  (pad "1" thru_hole circle (at 0 0 90) (size 1.4 1.4) (drill 0.7) (layers "*.Cu" "*.Mask") (remove_unused_layers no) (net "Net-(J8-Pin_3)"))
  (pad "2" thru_hole circle (at 5.08 0 90) (size 1.4 1.4) (drill 0.7) (layers "*.Cu" "*.Mask") (remove_unused_layers no) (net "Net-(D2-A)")))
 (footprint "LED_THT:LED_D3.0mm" (layer "F.Cu") (at 133.46 20)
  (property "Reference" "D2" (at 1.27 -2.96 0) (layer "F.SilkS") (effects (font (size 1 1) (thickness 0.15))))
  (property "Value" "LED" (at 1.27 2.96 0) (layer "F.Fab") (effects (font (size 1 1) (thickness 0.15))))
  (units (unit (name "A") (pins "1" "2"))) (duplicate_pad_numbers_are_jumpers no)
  (fp_line (start -0.29 -1.236) (end -0.29 -1.08) (stroke (width 0.12) (type solid)) (layer "F.SilkS"))
  (fp_line (start -0.29 1.08) (end -0.29 1.236) (stroke (width 0.12) (type solid)) (layer "F.SilkS"))
  (fp_arc (start -0.29 -1.235516) (mid 1.36566 -1.987699) (end 2.941437 -1.08) (stroke (width 0.12) (type solid)) (layer "F.SilkS"))
  (fp_arc (start 0.229039 -1.08) (mid 1.27 -1.5) (end 2.310961 -1.08) (stroke (width 0.12) (type solid)) (layer "F.SilkS"))
  (fp_arc (start 2.310961 1.08) (mid 1.27 1.5) (end 0.229039 1.08) (stroke (width 0.12) (type solid)) (layer "F.SilkS"))
  (fp_arc (start 2.941437 1.08) (mid 1.36566 1.987699) (end -0.29 1.235516) (stroke (width 0.12) (type solid)) (layer "F.SilkS"))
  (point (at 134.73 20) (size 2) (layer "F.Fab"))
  (pad "1" thru_hole rect (at 0 0) (size 1.8 1.8) (drill 0.9) (layers "*.Cu" "*.Mask") (remove_unused_layers no) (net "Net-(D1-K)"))
  (pad "2" thru_hole circle (at 2.54 0) (size 1.8 1.8) (drill 0.9) (layers "*.Cu" "*.Mask") (remove_unused_layers no) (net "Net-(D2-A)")))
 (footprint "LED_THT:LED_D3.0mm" (layer "F.Cu") (at 125.96 20)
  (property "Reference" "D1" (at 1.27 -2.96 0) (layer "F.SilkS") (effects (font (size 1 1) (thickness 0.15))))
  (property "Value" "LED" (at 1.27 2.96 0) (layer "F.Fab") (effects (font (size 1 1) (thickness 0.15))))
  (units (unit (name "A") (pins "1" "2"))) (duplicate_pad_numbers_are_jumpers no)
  (fp_line (start -0.29 -1.236) (end -0.29 -1.08) (stroke (width 0.12) (type solid)) (layer "F.SilkS"))
  (fp_line (start -0.29 1.08) (end -0.29 1.236) (stroke (width 0.12) (type solid)) (layer "F.SilkS"))
  (fp_arc (start -0.29 -1.235516) (mid 1.36566 -1.987699) (end 2.941437 -1.08) (stroke (width 0.12) (type solid)) (layer "F.SilkS"))
  (fp_arc (start 0.229039 -1.08) (mid 1.27 -1.5) (end 2.310961 -1.08) (stroke (width 0.12) (type solid)) (layer "F.SilkS"))
  (fp_arc (start 2.310961 1.08) (mid 1.27 1.5) (end 0.229039 1.08) (stroke (width 0.12) (type solid)) (layer "F.SilkS"))
  (fp_arc (start 2.941437 1.08) (mid 1.36566 1.987699) (end -0.29 1.235516) (stroke (width 0.12) (type solid)) (layer "F.SilkS"))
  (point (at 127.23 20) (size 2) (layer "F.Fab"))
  (pad "1" thru_hole rect (at 0 0) (size 1.8 1.8) (drill 0.9) (layers "*.Cu" "*.Mask") (remove_unused_layers no) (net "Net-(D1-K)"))
  (pad "2" thru_hole circle (at 2.54 0) (size 1.8 1.8) (drill 0.9) (layers "*.Cu" "*.Mask") (remove_unused_layers no) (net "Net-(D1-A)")))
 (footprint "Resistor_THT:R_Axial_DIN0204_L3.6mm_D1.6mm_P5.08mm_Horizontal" (layer "F.Cu") (at 130 31.04 90)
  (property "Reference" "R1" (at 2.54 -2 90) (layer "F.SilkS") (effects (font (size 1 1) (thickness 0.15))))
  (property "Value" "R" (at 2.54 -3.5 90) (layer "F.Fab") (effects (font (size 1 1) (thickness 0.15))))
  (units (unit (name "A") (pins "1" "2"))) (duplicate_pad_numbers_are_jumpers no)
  (fp_line (start 0.62 -0.92) (end 4.46 -0.92) (stroke (width 0.12) (type solid)) (layer "F.SilkS"))
  (fp_line (start 0.62 0.92) (end 4.46 0.92) (stroke (width 0.12) (type solid)) (layer "F.SilkS"))
  (pad "1" thru_hole circle (at 0 0 90) (size 1.4 1.4) (drill 0.7) (layers "*.Cu" "*.Mask") (remove_unused_layers no) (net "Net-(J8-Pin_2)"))
  (pad "2" thru_hole circle (at 5.08 0 90) (size 1.4 1.4) (drill 0.7) (layers "*.Cu" "*.Mask") (remove_unused_layers no) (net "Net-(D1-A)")))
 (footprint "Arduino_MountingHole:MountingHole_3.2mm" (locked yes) (layer "F.Cu") (at 113.97 97.46)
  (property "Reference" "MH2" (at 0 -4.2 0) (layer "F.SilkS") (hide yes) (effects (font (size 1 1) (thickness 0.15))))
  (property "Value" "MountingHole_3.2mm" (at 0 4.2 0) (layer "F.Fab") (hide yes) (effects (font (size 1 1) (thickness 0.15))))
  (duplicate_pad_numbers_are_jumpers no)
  (pad "" np_thru_hole circle (at 0 0) (size 3.2 3.2) (drill 3.2) (layers "*.Cu" "*.Mask")))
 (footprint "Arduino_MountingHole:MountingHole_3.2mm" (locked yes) (layer "F.Cu") (at 166.04 64.44)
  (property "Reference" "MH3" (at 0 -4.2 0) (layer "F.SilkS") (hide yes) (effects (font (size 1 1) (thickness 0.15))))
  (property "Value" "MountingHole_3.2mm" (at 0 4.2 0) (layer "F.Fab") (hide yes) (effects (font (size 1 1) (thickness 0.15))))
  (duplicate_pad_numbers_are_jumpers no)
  (pad "" np_thru_hole circle (at 0 0) (size 3.2 3.2) (drill 3.2) (layers "*.Cu" "*.Mask")))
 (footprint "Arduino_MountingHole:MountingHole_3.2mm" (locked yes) (layer "F.Cu") (at 166.04 92.38)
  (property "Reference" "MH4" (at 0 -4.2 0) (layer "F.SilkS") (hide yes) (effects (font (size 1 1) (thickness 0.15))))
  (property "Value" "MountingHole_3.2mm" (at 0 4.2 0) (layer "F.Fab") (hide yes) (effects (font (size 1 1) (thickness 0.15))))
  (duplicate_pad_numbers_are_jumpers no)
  (pad "" np_thru_hole circle (at 0 0) (size 3.2 3.2) (drill 3.2) (layers "*.Cu" "*.Mask")))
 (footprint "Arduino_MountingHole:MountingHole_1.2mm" (layer "F.Cu") (at 123.5 17)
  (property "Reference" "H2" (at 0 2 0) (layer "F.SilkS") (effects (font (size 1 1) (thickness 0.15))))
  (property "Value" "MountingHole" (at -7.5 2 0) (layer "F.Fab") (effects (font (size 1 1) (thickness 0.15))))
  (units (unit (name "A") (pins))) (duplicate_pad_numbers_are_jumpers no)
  (pad "" np_thru_hole circle (at 0 0) (size 1.2 1.2) (drill 1.2) (layers "*.Cu" "*.Mask")))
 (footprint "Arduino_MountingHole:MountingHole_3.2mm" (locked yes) (layer "F.Cu") (at 190.17 49.2)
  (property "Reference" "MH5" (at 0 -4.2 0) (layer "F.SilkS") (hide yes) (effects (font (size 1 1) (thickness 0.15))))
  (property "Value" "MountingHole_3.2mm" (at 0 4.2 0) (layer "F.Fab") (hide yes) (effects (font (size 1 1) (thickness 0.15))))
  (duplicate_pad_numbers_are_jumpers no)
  (pad "" np_thru_hole circle (at 0 0) (size 3.2 3.2) (drill 3.2) (layers "*.Cu" "*.Mask")))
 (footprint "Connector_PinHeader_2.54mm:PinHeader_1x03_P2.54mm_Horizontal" (layer "B.Cu") (at 128.42 35.115 -90)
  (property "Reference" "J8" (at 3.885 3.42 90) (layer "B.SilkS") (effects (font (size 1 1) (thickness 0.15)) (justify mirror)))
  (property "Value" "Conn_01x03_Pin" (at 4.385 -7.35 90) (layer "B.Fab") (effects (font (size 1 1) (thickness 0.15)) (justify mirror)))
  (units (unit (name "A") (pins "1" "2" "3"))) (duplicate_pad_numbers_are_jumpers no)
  (pad "1" thru_hole rect (at 0 0 270) (size 1.7 1.7) (drill 1) (layers "*.Cu" "*.Mask") (remove_unused_layers no) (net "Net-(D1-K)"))
  (pad "2" thru_hole circle (at 0 -2.54 270) (size 1.7 1.7) (drill 1) (layers "*.Cu" "*.Mask") (remove_unused_layers no)
   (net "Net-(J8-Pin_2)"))
  (pad "3" thru_hole circle (at 0 -5.08 270) (size 1.7 1.7) (drill 1) (layers "*.Cu" "*.Mask") (remove_unused_layers no)
   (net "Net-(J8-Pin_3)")))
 (gr_arc (start 100 47.422) (mid 100.223185 46.883185) (end 100.762 46.66) (stroke (width 0.15) (type solid)) (layer "Edge.Cuts"))
 (gr_line (start 100 99.238) (end 100 47.422) (stroke (width 0.15) (type solid)) (layer "Edge.Cuts"))
 (gr_line (start 100.762 46.66) (end 196.52 46.66) (stroke (width 0.15) (type solid)) (layer "Edge.Cuts"))
 (gr_arc (start 100.762 100) (mid 100.223185 99.776815) (end 100 99.238) (stroke (width 0.15) (type solid)) (layer "Edge.Cuts"))
 (gr_rect (start 122 15.5) (end 140 37.5) (stroke (width 0.15) (type default)) (fill no) (layer "Edge.Cuts"))
 (gr_line (start 196.52 46.66) (end 199.06 49.2) (stroke (width 0.15) (type solid)) (layer "Edge.Cuts"))
 (gr_line (start 198.298 100) (end 100.762 100) (stroke (width 0.15) (type solid)) (layer "Edge.Cuts"))
 (gr_line (start 199.06 49.2) (end 199.06 59.36) (stroke (width 0.15) (type solid)) (layer "Edge.Cuts"))
 (gr_line (start 199.06 59.36) (end 201.6 61.9) (stroke (width 0.15) (type solid)) (layer "Edge.Cuts"))
 (gr_line (start 199.06 98.73) (end 199.06 99.238) (stroke (width 0.15) (type solid)) (layer "Edge.Cuts"))
 (gr_arc (start 199.06 99.238) (mid 198.836815 99.776815) (end 198.298 100) (stroke (width 0.15) (type solid)) (layer "Edge.Cuts"))
 (gr_line (start 201.6 61.9) (end 201.6 96.19) (stroke (width 0.15) (type solid)) (layer "Edge.Cuts"))
 (gr_line (start 201.6 96.19) (end 199.06 98.73) (stroke (width 0.15) (type solid)) (layer "Edge.Cuts"))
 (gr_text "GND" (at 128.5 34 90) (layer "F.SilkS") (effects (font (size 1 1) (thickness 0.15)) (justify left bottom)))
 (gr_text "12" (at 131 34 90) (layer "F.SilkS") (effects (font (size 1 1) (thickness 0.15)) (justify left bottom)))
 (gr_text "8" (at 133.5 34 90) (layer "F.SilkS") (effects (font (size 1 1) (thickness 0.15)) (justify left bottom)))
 (segment (start 136 23) (end 136 20) (width 0.25) (layer "F.Cu") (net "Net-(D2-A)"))
 (segment (start 132.5 25.96) (end 133.04 25.96) (width 0.25) (layer "F.Cu") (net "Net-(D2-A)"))
 (segment (start 133.04 25.96) (end 136 23) (width 0.25) (layer "F.Cu") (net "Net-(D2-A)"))
 (segment (start 128.5 24.46) (end 128.5 20) (width 0.25) (layer "F.Cu") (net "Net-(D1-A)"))
 (segment (start 130 25.96) (end 128.5 24.46) (width 0.25) (layer "F.Cu") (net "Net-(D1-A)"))
 (segment (start 133.46 20) (end 132.235 18.775) (width 0.25) (layer "F.Cu") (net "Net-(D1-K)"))
 (segment (start 132.235 18.775) (end 127.185 18.775) (width 0.25) (layer "F.Cu") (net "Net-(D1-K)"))
 (segment (start 127.185 18.775) (end 125.96 20) (width 0.25) (layer "F.Cu") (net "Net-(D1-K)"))
 (segment (start 125.96 32.655) (end 128.42 35.115) (width 0.25) (layer "F.Cu") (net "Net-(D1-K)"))
 (segment (start 125.96 20) (end 125.96 32.655) (width 0.25) (layer "F.Cu") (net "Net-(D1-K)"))
 (segment (start 130 31.04) (end 130 34.155) (width 0.25) (layer "F.Cu") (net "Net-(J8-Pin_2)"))
 (segment (start 130 34.155) (end 130.96 35.115) (width 0.25) (layer "F.Cu") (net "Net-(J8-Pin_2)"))
 (segment (start 132.5 31.04) (end 132.5 34.115) (width 0.25) (layer "F.Cu") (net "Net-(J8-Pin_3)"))
 (segment (start 132.5 34.115) (end 133.5 35.115) (width 0.25) (layer "F.Cu") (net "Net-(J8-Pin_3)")))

